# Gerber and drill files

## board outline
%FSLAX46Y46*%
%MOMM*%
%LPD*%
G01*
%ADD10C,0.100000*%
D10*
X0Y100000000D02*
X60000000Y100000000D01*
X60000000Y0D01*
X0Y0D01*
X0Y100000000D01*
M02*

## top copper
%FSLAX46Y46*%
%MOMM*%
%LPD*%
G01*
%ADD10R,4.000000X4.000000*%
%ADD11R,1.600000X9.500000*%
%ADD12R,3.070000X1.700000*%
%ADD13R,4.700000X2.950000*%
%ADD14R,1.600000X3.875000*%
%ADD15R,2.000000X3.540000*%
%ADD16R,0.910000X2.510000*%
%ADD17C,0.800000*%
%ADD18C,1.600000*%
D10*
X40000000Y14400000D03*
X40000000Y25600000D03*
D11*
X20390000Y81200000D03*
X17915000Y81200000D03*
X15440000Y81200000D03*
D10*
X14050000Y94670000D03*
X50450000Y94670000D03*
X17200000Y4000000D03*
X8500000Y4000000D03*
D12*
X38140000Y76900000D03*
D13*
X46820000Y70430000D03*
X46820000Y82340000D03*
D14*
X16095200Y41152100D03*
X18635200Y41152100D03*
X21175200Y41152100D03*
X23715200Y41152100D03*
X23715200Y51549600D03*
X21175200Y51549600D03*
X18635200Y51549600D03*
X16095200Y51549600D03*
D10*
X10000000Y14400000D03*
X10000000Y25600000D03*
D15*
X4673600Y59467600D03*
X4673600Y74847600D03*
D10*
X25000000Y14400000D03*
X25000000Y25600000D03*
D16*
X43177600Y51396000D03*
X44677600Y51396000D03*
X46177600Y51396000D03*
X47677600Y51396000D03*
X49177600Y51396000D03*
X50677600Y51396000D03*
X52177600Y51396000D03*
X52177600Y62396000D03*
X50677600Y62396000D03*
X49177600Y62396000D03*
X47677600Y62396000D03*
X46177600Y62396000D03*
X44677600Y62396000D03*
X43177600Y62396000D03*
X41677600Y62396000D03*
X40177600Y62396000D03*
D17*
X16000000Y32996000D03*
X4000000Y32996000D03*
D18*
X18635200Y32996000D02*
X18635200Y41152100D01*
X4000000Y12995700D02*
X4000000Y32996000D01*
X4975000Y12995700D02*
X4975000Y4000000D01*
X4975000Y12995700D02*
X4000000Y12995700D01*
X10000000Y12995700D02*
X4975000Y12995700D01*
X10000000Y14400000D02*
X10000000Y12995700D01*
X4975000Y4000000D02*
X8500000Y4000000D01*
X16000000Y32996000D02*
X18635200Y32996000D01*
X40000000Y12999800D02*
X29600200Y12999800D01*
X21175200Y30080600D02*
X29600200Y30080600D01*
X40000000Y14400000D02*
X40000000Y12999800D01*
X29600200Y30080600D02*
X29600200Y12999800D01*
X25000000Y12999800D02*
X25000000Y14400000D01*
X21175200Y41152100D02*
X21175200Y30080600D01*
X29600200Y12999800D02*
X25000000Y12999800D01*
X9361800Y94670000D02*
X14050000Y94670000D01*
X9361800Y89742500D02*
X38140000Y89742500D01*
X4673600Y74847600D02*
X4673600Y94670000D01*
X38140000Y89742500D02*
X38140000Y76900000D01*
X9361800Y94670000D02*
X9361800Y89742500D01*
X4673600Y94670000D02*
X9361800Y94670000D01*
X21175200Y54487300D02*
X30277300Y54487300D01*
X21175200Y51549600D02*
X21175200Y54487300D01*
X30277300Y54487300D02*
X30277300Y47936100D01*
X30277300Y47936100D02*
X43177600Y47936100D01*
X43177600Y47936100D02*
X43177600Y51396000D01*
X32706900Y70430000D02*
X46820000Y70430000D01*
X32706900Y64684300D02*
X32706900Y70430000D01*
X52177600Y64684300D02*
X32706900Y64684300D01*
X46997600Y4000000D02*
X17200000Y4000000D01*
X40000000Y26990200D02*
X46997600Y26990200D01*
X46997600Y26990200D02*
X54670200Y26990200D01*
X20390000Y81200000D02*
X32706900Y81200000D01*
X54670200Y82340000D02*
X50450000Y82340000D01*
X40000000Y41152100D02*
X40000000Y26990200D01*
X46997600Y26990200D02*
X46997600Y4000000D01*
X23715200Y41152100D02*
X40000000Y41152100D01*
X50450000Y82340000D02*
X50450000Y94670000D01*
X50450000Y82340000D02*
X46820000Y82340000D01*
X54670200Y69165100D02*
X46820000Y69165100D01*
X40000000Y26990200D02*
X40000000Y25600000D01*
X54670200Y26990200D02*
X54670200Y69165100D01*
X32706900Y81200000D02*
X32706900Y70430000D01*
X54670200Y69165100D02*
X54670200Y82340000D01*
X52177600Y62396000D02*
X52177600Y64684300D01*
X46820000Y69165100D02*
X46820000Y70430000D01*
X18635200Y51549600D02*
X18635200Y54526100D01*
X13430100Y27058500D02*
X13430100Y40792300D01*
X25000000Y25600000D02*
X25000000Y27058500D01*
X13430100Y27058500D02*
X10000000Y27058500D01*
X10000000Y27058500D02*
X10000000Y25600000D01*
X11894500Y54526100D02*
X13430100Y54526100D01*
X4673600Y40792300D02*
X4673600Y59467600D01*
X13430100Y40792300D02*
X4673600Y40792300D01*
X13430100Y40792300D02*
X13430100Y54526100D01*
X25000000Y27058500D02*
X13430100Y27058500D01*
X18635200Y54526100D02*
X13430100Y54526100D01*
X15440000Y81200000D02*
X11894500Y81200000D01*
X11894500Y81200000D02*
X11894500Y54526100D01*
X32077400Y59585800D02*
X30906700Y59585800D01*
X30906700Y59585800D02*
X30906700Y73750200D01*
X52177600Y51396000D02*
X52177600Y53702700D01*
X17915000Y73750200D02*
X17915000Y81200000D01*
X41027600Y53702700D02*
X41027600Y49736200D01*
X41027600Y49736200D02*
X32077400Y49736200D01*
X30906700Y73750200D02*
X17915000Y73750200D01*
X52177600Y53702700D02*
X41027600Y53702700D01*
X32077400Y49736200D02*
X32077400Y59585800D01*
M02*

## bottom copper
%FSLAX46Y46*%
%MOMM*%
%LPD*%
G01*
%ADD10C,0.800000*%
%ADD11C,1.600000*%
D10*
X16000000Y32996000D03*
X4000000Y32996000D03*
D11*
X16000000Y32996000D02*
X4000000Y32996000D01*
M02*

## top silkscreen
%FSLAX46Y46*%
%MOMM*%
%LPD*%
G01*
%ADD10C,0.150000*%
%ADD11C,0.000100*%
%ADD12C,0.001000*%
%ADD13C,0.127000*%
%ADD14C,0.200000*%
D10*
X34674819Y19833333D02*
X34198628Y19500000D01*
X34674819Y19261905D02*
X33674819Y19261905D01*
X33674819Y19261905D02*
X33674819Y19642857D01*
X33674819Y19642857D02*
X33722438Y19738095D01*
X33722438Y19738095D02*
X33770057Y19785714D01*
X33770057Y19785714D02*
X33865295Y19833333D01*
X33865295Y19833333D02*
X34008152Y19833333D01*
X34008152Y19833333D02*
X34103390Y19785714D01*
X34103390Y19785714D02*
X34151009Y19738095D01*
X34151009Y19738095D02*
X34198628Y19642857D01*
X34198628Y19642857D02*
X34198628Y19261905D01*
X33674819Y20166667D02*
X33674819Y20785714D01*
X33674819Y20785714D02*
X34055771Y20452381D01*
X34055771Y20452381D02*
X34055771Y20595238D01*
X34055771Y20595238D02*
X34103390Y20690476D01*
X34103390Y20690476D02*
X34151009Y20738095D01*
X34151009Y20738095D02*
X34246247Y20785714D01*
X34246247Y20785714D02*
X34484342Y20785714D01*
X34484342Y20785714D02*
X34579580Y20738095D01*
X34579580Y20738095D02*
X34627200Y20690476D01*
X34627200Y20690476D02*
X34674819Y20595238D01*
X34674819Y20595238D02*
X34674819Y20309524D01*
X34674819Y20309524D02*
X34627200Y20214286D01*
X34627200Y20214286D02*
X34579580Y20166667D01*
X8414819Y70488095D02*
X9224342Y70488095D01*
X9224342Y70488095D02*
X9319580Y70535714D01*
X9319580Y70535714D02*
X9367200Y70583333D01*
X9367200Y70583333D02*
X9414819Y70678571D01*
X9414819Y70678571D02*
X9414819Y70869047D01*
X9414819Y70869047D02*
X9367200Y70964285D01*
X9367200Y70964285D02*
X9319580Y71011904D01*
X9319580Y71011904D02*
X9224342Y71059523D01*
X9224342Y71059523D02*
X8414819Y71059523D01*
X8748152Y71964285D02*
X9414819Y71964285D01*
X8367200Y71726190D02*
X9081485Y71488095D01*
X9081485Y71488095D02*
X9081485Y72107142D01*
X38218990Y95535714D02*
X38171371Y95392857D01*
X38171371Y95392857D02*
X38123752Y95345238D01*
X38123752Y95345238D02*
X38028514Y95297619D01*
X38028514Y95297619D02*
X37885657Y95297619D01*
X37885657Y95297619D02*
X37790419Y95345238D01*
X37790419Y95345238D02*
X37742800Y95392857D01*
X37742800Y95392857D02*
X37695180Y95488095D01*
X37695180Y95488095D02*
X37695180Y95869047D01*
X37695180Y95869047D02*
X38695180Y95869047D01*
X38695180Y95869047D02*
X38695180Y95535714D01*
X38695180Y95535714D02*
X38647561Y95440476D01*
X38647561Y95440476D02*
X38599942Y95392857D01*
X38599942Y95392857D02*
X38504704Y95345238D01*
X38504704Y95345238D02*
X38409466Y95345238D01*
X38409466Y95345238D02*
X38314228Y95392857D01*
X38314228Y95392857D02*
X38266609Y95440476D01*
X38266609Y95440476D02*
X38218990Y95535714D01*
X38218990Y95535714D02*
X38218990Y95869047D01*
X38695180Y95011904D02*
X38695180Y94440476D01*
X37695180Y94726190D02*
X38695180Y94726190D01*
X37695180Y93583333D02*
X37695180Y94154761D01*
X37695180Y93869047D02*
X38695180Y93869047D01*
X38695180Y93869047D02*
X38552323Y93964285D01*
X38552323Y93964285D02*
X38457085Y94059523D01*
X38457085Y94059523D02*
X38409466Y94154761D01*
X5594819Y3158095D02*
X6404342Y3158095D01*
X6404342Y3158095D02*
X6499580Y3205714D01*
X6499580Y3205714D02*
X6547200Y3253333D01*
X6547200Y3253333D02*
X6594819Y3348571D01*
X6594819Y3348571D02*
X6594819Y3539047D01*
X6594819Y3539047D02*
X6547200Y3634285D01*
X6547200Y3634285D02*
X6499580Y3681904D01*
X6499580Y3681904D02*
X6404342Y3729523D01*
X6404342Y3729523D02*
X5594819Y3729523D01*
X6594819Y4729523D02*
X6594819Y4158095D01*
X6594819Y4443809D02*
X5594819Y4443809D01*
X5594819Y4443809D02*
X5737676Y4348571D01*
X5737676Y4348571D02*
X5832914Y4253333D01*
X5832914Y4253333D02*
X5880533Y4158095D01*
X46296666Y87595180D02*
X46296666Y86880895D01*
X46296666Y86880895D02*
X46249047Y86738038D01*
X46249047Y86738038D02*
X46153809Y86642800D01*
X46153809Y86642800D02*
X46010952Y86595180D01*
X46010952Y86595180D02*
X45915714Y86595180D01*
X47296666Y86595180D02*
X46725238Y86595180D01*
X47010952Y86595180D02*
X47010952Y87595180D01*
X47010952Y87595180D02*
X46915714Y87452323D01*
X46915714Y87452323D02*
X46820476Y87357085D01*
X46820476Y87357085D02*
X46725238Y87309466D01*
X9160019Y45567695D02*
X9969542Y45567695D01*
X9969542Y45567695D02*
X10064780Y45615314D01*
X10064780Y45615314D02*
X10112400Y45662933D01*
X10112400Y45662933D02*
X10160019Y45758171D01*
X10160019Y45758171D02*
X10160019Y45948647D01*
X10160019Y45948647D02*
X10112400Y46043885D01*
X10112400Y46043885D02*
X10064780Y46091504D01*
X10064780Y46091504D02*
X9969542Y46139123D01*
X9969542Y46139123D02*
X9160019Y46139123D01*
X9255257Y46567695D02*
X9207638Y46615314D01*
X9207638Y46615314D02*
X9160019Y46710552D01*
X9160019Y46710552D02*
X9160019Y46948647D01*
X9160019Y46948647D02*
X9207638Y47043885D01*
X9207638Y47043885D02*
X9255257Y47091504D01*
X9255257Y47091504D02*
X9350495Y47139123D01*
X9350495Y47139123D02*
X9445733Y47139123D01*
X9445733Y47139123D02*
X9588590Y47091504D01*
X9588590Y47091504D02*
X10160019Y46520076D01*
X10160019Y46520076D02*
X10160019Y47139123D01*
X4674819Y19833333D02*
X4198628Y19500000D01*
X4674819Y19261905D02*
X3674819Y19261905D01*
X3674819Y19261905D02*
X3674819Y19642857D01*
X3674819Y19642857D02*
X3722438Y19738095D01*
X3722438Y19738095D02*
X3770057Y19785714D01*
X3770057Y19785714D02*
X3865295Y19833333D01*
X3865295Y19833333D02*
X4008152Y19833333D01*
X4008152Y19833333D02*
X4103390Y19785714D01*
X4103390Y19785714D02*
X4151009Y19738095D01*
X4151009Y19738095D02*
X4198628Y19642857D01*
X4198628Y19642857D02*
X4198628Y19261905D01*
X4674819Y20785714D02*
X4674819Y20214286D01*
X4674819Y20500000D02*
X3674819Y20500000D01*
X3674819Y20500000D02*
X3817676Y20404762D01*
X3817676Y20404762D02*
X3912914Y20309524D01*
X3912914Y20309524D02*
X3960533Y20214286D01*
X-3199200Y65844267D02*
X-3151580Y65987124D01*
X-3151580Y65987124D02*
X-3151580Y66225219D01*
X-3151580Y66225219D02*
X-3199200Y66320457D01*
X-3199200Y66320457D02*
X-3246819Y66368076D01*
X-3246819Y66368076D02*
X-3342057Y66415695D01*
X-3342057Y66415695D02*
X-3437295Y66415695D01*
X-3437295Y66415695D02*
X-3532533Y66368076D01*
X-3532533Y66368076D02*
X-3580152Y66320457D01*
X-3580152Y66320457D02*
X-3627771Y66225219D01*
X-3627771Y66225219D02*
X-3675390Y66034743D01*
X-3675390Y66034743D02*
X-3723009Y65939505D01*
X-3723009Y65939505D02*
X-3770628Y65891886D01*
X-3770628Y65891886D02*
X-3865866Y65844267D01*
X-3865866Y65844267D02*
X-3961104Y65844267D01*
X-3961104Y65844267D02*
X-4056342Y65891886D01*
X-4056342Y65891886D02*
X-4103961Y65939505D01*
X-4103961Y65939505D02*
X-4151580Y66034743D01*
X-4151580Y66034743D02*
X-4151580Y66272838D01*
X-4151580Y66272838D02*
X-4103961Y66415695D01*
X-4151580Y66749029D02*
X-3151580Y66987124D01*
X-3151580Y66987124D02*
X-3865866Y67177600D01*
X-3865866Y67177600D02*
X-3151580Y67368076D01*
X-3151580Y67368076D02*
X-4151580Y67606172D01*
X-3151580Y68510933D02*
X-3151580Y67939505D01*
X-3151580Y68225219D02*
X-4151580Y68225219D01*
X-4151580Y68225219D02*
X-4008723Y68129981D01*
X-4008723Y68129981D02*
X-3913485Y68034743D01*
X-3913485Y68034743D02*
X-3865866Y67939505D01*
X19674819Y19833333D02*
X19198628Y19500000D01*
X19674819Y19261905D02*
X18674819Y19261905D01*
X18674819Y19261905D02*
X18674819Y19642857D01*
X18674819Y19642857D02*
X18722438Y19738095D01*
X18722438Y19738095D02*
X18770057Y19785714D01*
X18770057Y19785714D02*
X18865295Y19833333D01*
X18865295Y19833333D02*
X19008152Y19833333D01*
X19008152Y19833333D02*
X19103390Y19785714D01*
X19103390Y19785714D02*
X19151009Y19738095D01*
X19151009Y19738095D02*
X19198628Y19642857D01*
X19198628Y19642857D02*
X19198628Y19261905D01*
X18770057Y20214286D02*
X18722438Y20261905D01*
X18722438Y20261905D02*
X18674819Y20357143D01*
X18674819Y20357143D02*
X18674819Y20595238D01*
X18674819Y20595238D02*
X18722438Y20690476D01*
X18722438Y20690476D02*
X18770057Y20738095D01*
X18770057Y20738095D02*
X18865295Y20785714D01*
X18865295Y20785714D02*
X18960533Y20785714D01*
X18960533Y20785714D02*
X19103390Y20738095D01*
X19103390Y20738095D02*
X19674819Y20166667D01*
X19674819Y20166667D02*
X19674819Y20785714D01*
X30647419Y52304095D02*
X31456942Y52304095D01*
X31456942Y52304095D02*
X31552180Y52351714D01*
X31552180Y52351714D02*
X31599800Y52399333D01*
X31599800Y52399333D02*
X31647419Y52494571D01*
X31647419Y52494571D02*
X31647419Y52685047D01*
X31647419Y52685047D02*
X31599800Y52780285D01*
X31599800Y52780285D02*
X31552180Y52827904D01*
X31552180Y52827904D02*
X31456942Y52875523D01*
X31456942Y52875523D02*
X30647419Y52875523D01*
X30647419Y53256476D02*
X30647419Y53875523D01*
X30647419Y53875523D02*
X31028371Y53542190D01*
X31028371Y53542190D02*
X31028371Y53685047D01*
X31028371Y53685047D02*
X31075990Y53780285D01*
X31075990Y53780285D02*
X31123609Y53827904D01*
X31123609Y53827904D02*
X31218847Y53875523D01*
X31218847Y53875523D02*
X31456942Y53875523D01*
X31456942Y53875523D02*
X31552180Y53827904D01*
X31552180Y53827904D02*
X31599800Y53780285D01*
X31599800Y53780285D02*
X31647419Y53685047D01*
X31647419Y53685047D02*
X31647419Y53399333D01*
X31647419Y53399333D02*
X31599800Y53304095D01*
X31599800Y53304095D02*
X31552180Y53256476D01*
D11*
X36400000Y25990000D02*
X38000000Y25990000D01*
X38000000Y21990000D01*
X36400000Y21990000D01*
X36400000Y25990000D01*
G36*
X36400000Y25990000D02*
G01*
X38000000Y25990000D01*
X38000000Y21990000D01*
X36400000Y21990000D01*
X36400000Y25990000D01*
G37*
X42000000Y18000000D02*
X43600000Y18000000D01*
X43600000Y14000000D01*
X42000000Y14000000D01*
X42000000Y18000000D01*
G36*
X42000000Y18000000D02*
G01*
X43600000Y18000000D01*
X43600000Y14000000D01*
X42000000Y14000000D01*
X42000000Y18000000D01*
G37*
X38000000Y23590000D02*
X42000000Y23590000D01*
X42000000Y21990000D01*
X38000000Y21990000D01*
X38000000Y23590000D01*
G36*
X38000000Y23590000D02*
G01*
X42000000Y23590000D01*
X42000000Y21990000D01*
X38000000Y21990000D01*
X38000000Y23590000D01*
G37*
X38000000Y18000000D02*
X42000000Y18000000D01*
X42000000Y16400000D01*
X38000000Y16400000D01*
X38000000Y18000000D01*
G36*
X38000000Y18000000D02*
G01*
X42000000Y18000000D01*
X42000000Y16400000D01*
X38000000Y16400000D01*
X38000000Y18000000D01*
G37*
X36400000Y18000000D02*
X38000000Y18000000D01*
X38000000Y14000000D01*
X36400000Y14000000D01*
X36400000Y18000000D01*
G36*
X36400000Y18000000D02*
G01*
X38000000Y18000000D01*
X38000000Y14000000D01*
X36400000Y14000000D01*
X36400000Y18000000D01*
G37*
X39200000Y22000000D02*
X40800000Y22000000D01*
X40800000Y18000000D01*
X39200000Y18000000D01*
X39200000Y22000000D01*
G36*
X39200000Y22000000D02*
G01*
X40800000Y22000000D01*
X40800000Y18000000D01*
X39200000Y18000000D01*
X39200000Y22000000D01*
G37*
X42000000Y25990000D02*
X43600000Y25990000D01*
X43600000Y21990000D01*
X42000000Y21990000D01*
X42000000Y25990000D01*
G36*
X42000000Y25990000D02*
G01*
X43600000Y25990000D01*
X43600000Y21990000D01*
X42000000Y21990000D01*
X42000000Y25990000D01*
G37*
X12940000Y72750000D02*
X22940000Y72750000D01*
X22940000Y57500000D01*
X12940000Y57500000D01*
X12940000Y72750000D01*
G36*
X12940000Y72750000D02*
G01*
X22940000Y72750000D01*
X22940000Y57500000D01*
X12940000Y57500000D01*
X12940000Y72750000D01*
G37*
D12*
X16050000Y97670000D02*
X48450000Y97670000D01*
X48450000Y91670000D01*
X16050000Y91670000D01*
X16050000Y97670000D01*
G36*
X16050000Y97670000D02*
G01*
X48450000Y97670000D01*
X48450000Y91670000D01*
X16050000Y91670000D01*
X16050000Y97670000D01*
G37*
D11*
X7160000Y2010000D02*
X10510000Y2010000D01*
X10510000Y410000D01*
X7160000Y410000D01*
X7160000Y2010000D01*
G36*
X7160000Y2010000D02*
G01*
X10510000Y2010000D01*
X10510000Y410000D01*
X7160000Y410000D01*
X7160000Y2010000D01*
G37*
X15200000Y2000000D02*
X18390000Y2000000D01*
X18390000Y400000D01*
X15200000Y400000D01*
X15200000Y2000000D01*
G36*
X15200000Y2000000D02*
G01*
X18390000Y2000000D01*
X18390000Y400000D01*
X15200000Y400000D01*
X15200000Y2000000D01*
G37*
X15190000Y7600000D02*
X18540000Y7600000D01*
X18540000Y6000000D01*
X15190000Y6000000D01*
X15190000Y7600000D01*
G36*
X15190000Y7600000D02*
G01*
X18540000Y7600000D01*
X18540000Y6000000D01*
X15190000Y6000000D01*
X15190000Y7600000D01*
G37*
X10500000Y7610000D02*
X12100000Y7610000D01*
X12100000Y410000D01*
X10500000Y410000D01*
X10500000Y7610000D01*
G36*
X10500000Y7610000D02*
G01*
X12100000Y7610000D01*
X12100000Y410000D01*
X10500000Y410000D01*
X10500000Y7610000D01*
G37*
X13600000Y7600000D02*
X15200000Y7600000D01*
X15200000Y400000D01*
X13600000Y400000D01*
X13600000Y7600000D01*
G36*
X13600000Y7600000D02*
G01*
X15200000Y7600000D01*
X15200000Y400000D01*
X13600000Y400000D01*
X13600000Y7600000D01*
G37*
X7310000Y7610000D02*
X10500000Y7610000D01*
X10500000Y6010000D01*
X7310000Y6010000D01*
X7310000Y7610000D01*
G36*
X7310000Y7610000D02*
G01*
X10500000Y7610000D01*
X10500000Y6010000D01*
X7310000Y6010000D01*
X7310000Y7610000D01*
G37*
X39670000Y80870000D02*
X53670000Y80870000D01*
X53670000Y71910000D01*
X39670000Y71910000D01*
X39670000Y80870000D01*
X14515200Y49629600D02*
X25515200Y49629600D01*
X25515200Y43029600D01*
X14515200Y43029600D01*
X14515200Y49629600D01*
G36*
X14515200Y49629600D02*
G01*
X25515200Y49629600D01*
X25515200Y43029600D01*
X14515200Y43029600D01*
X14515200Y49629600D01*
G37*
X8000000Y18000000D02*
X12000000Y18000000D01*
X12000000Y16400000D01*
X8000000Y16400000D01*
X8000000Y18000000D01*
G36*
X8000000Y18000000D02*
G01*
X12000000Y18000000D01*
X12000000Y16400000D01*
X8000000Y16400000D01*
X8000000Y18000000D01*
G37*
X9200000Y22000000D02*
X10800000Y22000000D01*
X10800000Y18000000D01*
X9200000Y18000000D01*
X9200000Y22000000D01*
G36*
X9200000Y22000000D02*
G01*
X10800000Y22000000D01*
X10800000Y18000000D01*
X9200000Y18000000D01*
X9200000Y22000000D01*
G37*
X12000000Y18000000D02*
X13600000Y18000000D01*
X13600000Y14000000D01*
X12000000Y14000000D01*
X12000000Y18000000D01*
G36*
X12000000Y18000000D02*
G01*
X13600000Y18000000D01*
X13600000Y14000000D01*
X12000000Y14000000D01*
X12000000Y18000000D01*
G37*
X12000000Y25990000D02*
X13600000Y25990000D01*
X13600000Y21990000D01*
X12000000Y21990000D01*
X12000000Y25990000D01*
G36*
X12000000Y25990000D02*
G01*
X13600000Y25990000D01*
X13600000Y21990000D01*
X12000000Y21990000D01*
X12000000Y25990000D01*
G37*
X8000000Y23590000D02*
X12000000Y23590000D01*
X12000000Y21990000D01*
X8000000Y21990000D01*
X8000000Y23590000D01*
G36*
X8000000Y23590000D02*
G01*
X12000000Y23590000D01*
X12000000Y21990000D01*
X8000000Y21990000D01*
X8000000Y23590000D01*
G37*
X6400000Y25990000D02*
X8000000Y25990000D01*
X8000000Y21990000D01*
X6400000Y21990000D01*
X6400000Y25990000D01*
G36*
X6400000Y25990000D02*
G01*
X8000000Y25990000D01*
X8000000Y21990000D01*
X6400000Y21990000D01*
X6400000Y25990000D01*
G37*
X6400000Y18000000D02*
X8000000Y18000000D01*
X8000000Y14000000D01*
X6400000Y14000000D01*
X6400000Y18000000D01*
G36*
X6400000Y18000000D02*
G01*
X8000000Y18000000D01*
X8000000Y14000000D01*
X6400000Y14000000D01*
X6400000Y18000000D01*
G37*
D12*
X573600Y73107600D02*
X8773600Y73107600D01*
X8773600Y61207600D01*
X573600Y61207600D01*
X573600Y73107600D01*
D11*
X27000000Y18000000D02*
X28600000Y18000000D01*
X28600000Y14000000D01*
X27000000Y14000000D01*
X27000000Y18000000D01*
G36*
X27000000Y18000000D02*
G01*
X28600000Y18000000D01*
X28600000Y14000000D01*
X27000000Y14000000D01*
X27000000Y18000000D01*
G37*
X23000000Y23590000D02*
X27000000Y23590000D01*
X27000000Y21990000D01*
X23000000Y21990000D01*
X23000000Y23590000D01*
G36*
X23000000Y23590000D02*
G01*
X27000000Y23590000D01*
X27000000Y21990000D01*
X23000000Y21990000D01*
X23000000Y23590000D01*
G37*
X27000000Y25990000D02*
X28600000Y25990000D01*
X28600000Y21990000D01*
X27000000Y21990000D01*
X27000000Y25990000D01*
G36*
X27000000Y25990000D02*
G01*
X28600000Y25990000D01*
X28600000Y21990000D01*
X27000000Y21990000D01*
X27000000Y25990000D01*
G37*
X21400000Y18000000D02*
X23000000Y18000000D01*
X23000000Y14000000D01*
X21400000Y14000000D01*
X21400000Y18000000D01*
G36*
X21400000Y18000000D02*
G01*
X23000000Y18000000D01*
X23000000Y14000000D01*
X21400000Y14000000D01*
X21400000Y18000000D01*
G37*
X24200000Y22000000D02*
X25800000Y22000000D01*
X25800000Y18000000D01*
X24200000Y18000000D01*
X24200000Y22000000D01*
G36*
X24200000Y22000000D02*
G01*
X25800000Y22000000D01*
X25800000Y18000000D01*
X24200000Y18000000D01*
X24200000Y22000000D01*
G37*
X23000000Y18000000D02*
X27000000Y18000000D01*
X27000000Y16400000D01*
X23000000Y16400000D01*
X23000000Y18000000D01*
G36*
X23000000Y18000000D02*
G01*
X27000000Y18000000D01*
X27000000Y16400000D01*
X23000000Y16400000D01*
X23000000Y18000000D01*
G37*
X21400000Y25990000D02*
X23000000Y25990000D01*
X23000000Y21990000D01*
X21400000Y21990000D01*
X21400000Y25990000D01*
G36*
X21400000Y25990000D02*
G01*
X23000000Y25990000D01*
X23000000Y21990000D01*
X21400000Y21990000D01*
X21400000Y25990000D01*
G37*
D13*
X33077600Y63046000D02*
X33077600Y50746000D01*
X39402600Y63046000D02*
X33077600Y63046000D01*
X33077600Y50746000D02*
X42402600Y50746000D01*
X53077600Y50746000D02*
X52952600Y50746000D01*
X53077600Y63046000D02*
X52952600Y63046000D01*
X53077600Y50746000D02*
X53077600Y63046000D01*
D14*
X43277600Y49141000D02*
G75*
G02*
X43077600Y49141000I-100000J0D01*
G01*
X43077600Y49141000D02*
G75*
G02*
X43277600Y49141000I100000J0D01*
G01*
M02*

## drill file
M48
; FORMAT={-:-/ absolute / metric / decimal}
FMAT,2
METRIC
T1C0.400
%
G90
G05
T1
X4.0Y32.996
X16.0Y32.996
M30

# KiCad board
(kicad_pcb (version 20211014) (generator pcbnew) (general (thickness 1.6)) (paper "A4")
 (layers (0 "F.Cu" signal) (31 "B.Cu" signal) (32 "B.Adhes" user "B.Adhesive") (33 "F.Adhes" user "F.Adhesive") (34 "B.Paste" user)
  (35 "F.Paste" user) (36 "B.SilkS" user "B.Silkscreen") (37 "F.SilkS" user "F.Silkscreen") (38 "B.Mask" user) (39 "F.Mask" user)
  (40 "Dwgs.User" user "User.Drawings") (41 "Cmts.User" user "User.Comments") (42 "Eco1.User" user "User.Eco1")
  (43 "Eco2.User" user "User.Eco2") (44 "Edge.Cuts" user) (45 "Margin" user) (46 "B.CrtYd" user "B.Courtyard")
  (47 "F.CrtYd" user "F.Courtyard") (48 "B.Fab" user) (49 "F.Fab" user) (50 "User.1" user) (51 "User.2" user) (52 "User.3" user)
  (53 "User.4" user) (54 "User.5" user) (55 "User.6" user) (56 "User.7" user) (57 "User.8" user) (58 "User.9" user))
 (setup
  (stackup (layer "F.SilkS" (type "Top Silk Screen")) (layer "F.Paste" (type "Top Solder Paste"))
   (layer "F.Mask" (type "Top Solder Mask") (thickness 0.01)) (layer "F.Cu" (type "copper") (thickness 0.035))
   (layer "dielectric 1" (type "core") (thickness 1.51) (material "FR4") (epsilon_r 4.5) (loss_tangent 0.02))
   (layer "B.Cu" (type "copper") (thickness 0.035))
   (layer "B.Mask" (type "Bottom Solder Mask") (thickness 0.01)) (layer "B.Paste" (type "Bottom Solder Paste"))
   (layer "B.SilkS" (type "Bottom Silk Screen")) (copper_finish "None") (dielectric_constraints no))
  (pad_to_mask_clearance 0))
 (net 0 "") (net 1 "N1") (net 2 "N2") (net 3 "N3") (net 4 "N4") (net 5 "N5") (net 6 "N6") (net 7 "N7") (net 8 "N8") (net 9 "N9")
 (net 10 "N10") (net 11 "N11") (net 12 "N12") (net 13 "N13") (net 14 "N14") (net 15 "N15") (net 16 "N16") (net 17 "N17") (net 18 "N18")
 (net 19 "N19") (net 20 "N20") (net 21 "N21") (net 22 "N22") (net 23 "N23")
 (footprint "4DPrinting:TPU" (layer "F.Cu") (at 40 -20 90)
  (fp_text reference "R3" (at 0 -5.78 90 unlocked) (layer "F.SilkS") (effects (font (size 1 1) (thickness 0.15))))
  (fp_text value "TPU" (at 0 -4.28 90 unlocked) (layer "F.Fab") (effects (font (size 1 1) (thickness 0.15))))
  (fp_rect (start 1.99 -3.6) (end 5.99 -2) (layer "F.SilkS") (width 0.0001) (fill solid))
  (fp_rect (start -6 2) (end -2 3.6) (layer "F.SilkS") (width 0.0001) (fill solid))
  (fp_rect (start 1.99 -2) (end 3.59 2) (layer "F.SilkS") (width 0.0001) (fill solid))
  (fp_rect (start -3.6 -2) (end -2 2) (layer "F.SilkS") (width 0.0001) (fill solid))
  (fp_rect (start -6 -3.6) (end -2 -2) (layer "F.SilkS") (width 0.0001) (fill solid))
  (fp_rect (start -2 -0.8) (end 2 0.8) (layer "F.SilkS") (width 0.0001) (fill solid))
  (fp_rect (start 1.99 2) (end 5.99 3.6) (layer "F.SilkS") (width 0.0001) (fill solid))
  (pad "1" smd rect (at -5.6 0 90) (size 4 4) (layers "F.Cu" "F.Paste" "F.Mask") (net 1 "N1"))
  (pad "2" smd rect (at 5.6 0 90) (size 4 4) (layers "F.Cu" "F.Paste" "F.Mask") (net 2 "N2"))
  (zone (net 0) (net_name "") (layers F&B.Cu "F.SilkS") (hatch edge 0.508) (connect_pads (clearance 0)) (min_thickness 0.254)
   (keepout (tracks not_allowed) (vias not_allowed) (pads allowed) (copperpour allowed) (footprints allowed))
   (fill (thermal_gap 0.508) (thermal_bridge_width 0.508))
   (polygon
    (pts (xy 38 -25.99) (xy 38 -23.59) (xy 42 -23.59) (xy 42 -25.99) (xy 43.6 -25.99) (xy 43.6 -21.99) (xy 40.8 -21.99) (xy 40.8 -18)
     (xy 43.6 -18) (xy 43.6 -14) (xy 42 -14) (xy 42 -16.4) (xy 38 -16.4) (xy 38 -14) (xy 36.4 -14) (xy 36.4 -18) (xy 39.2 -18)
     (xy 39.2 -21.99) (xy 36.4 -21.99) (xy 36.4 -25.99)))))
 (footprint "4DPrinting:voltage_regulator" (layer "F.Cu") (at 17.99 -71.23 90)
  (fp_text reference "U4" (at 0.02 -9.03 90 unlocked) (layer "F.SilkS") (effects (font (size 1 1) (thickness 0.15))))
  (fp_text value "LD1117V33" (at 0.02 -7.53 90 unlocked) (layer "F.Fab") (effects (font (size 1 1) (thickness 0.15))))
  (fp_rect (start -13.73 -5.05) (end 1.52 4.95) (layer "F.SilkS") (width 0.0001) (fill solid))
  (pad "1" smd rect (at 9.97 2.4 90) (size 9.5 1.6) (layers "F.Cu" "F.Paste" "F.Mask") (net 2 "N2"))
  (pad "2" smd rect (at 9.97 -0.075 90) (size 9.5 1.6) (layers "F.Cu" "F.Paste" "F.Mask") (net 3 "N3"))
  (pad "3" smd rect (at 9.97 -2.55 90) (size 9.5 1.6) (layers "F.Cu" "F.Paste" "F.Mask") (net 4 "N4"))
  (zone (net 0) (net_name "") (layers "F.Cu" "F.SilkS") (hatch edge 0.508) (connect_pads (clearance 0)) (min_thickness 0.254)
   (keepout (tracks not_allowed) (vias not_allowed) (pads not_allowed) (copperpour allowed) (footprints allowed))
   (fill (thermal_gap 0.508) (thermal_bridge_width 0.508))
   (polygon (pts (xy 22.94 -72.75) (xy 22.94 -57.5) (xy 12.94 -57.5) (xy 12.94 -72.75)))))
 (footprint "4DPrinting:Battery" (layer "F.Cu") (at 32.25 -94.67 -90)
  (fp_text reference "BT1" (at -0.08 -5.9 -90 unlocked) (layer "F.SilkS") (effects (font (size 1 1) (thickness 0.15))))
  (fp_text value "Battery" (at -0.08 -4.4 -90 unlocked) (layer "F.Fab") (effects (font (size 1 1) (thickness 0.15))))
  (fp_rect (start -3 -16.2) (end 3 16.2) (layer "F.SilkS") (width 0.001) (fill solid))
  (pad "1" smd rect (at 0 18.2 270) (size 4 4) (layers "F.Cu" "F.Paste" "F.Mask") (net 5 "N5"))
  (pad "2" smd rect (at 0 -18.2 270) (size 4 4) (layers "F.Cu" "F.Paste" "F.Mask") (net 2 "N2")))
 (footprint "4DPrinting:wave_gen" (layer "F.Cu") (at 12.85 -4 90)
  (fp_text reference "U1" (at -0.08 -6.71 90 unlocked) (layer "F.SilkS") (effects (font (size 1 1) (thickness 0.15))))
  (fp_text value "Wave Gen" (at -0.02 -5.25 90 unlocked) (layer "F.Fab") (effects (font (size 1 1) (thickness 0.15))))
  (fp_rect (start -3.59 -2.34) (end -1.99 -5.69) (layer "F.SilkS") (width 0.0001) (fill solid))
  (fp_rect (start -2 2.35) (end -3.6 5.54) (layer "F.SilkS") (width 0.0001) (fill solid))
  (fp_rect (start 3.6 2.34) (end 2 5.69) (layer "F.SilkS") (width 0.0001) (fill solid))
  (fp_rect (start 3.61 -0.75) (end -3.59 -2.35) (layer "F.SilkS") (width 0.0001) (fill solid))
  (fp_rect (start -3.6 0.75) (end 3.6 2.35) (layer "F.SilkS") (width 0.0001) (fill solid))
  (fp_rect (start 2.01 -2.35) (end 3.61 -5.54) (layer "F.SilkS") (width 0.0001) (fill solid))
  (pad "1" smd rect (at 0 4.35 90) (size 4 4) (layers "F.Cu" "F.Paste" "F.Mask") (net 2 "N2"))
  (pad "2" smd rect (at 0 -4.35 270) (size 4 4) (layers "F.Cu" "F.Paste" "F.Mask") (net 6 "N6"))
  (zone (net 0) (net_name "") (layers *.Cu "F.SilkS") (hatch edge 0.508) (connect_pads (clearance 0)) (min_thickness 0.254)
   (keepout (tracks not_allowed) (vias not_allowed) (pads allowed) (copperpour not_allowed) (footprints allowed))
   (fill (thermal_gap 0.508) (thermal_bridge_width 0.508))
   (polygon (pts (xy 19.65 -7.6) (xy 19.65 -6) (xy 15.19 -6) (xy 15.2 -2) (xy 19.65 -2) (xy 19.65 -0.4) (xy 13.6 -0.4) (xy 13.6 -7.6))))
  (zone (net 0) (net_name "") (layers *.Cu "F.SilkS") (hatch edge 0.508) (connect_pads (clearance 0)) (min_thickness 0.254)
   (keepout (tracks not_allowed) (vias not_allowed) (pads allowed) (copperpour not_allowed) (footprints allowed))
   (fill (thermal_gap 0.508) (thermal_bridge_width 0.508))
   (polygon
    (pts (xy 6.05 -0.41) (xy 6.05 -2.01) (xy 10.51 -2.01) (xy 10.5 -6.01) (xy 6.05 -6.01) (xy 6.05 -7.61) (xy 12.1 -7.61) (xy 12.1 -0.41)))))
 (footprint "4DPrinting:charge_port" (layer "F.Cu") (at 46.67 -76.39)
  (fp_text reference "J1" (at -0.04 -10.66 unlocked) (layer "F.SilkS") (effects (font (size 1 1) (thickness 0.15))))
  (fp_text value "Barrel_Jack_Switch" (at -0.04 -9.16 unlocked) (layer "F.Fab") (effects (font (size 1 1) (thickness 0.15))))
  (fp_rect (start -7 -4.48) (end 7 4.48) (layer "F.SilkS") (width 0.0001) (fill none))
  (pad "1" smd rect (at -8.53 -0.51 180) (size 3.07 1.7) (layers "F.Cu" "F.Paste" "F.Mask") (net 5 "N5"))
  (pad "2" smd rect (at 0.15 5.96 180) (size 4.7 2.95) (layers "F.Cu" "F.Paste" "F.Mask") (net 2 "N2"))
  (pad "3" smd rect (at 0.15 -5.95 180) (size 4.7 2.95) (layers "F.Cu" "F.Paste" "F.Mask") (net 2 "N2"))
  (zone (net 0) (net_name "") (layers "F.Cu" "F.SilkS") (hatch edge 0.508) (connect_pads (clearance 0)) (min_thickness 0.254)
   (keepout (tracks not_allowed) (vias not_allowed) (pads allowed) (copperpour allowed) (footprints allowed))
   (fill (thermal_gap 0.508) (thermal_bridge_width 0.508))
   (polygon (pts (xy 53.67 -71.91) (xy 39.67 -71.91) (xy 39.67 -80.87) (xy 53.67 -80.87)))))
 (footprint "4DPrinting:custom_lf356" (layer "F.Cu") (at 20.0152 -46.3296 90)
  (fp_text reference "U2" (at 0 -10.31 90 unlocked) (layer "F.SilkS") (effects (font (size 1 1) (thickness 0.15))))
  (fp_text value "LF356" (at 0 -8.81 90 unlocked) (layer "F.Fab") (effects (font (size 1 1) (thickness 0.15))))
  (fp_rect (start -3.3 -5.5) (end 3.3 5.5) (layer "F.SilkS") (width 0.0001) (fill solid))
  (pad "1" smd rect (at -5.1775 -3.92 90) (size 3.875 1.6) (layers "F.Cu" "F.Paste" "F.Mask") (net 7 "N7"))
  (pad "2" smd rect (at -5.1775 -1.38 90) (size 3.875 1.6) (layers "F.Cu" "F.Paste" "F.Mask") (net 6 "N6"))
  (pad "3" smd rect (at -5.1775 1.16 90) (size 3.875 1.6) (layers "F.Cu" "F.Paste" "F.Mask") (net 1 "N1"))
  (pad "4" smd rect (at -5.1775 3.7 90) (size 3.875 1.6) (layers "F.Cu" "F.Paste" "F.Mask") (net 2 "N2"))
  (pad "5" smd rect (at 5.22 3.7 90) (size 3.875 1.6) (layers "F.Cu" "F.Paste" "F.Mask") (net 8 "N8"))
  (pad "6" smd rect (at 5.22 1.16 90) (size 3.875 1.6) (layers "F.Cu" "F.Paste" "F.Mask") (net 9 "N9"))
  (pad "7" smd rect (at 5.22 -1.38 90) (size 3.875 1.6) (layers "F.Cu" "F.Paste" "F.Mask") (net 4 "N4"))
  (pad "8" smd rect (at 5.22 -3.92 90) (size 3.875 1.6) (layers "F.Cu" "F.Paste" "F.Mask") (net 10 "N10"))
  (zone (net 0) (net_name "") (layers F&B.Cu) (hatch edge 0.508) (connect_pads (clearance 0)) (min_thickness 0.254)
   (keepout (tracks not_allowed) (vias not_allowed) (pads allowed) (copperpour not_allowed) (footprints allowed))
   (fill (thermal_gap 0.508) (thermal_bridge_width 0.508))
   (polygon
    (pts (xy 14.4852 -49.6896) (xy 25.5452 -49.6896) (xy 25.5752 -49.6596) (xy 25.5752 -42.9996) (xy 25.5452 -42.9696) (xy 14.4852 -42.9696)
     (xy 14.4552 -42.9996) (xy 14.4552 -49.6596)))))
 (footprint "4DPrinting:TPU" (layer "F.Cu") (at 10 -20 90)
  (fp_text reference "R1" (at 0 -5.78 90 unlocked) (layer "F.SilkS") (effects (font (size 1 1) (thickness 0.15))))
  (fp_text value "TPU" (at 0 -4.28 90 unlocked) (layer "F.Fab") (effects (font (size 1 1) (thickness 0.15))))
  (fp_rect (start -3.6 -2) (end -2 2) (layer "F.SilkS") (width 0.0001) (fill solid))
  (fp_rect (start -2 -0.8) (end 2 0.8) (layer "F.SilkS") (width 0.0001) (fill solid))
  (fp_rect (start -6 2) (end -2 3.6) (layer "F.SilkS") (width 0.0001) (fill solid))
  (fp_rect (start 1.99 2) (end 5.99 3.6) (layer "F.SilkS") (width 0.0001) (fill solid))
  (fp_rect (start 1.99 -2) (end 3.59 2) (layer "F.SilkS") (width 0.0001) (fill solid))
  (fp_rect (start 1.99 -3.6) (end 5.99 -2) (layer "F.SilkS") (width 0.0001) (fill solid))
  (fp_rect (start -6 -3.6) (end -2 -2) (layer "F.SilkS") (width 0.0001) (fill solid))
  (pad "1" smd rect (at -5.6 0 90) (size 4 4) (layers "F.Cu" "F.Paste" "F.Mask") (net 6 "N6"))
  (pad "2" smd rect (at 5.6 0 90) (size 4 4) (layers "F.Cu" "F.Paste" "F.Mask") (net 4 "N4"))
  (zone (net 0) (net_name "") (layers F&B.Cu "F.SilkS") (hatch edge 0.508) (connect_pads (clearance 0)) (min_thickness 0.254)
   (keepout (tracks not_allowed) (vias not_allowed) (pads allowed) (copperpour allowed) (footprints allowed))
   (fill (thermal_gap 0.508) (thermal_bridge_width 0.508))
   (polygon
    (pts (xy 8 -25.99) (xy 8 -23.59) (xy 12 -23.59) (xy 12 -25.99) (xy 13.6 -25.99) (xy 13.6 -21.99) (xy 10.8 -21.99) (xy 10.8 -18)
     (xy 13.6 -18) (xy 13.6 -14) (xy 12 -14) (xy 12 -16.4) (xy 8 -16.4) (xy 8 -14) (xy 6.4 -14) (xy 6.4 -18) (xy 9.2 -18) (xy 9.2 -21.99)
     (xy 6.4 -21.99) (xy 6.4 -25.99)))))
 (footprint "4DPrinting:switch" (layer "F.Cu") (at 4.6736 -67.1576 90)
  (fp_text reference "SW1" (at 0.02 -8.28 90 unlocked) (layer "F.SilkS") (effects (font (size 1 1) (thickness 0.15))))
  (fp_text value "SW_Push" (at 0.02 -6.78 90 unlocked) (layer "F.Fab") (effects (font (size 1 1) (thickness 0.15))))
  (fp_rect (start -5.95 4.1) (end 5.95 -4.1) (layer "F.SilkS") (width 0.001) (fill none))
  (pad "1" smd rect (at -7.69 0 90) (size 3.54 2) (layers "F.Cu" "F.Paste" "F.Mask") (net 4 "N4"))
  (pad "2" smd rect (at 7.69 0 90) (size 3.54 2) (layers "F.Cu" "F.Paste" "F.Mask") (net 5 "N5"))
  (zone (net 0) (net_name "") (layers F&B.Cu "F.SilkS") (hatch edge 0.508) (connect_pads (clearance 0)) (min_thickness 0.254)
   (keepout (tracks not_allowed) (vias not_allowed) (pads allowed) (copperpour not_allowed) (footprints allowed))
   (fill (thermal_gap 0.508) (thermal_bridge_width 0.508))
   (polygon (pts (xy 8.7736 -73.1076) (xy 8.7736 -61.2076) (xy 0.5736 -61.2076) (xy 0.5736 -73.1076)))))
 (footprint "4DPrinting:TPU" (layer "F.Cu") (at 25 -20 90)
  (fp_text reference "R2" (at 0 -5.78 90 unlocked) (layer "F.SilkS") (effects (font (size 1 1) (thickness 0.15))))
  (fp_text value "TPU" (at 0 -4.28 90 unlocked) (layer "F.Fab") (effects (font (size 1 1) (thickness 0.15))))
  (fp_rect (start -6 2) (end -2 3.6) (layer "F.SilkS") (width 0.0001) (fill solid))
  (fp_rect (start 1.99 -2) (end 3.59 2) (layer "F.SilkS") (width 0.0001) (fill solid))
  (fp_rect (start 1.99 2) (end 5.99 3.6) (layer "F.SilkS") (width 0.0001) (fill solid))
  (fp_rect (start -6 -3.6) (end -2 -2) (layer "F.SilkS") (width 0.0001) (fill solid))
  (fp_rect (start -2 -0.8) (end 2 0.8) (layer "F.SilkS") (width 0.0001) (fill solid))
  (fp_rect (start -3.6 -2) (end -2 2) (layer "F.SilkS") (width 0.0001) (fill solid))
  (fp_rect (start 1.99 -3.6) (end 5.99 -2) (layer "F.SilkS") (width 0.0001) (fill solid))
  (pad "1" smd rect (at -5.6 0 90) (size 4 4) (layers "F.Cu" "F.Paste" "F.Mask") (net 1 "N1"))
  (pad "2" smd rect (at 5.6 0 90) (size 4 4) (layers "F.Cu" "F.Paste" "F.Mask") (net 4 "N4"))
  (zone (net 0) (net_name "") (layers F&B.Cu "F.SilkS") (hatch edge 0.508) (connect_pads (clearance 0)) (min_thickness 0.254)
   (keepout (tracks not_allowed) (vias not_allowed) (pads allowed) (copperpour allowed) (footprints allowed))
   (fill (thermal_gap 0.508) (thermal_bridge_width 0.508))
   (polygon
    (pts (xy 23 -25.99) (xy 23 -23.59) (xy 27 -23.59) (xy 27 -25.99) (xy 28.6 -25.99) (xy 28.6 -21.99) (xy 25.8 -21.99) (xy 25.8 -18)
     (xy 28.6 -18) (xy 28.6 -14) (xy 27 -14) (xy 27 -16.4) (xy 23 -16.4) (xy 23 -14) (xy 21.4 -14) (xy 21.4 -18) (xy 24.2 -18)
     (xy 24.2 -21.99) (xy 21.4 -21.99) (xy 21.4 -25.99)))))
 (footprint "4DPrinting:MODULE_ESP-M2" (layer "F.Cu") (at 43.0776 -56.896 90)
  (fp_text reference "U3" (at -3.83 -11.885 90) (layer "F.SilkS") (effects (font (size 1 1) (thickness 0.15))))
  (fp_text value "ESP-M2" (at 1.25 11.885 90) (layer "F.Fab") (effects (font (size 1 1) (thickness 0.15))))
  (fp_line (start 6.15 -10) (end -6.15 -10) (layer "F.SilkS") (width 0.127))
  (fp_line (start 6.15 -3.675) (end 6.15 -10) (layer "F.SilkS") (width 0.127))
  (fp_line (start -6.15 -10) (end -6.15 -0.675) (layer "F.SilkS") (width 0.127))
  (fp_line (start -6.15 10) (end -6.15 9.875) (layer "F.SilkS") (width 0.127))
  (fp_line (start 6.15 10) (end 6.15 9.875) (layer "F.SilkS") (width 0.127))
  (fp_line (start -6.15 10) (end 6.15 10) (layer "F.SilkS") (width 0.127))
  (fp_circle (center -7.755 0.1) (end -7.655 0.1) (layer "F.SilkS") (width 0.2) (fill none))
  (pad "1" smd rect (at -5.5 0.1 90) (size 2.51 0.91) (layers "F.Cu" "F.Paste" "F.Mask") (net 9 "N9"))
  (pad "2" smd rect (at -5.5 1.6 90) (size 2.51 0.91) (layers "F.Cu" "F.Paste" "F.Mask") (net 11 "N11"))
  (pad "3" smd rect (at -5.5 3.1 90) (size 2.51 0.91) (layers "F.Cu" "F.Paste" "F.Mask") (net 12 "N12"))
  (pad "4" smd rect (at -5.5 4.6 90) (size 2.51 0.91) (layers "F.Cu" "F.Paste" "F.Mask") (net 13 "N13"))
  (pad "5" smd rect (at -5.5 6.1 90) (size 2.51 0.91) (layers "F.Cu" "F.Paste" "F.Mask") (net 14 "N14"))
  (pad "6" smd rect (at -5.5 7.6 90) (size 2.51 0.91) (layers "F.Cu" "F.Paste" "F.Mask") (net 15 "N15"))
  (pad "7" smd rect (at -5.5 9.1 90) (size 2.51 0.91) (layers "F.Cu" "F.Paste" "F.Mask") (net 3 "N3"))
  (pad "8" smd rect (at 5.5 9.1 90) (size 2.51 0.91) (layers "F.Cu" "F.Paste" "F.Mask") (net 2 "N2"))
  (pad "9" smd rect (at 5.5 7.6 90) (size 2.51 0.91) (layers "F.Cu" "F.Paste" "F.Mask") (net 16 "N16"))
  (pad "10" smd rect (at 5.5 6.1 90) (size 2.51 0.91) (layers "F.Cu" "F.Paste" "F.Mask") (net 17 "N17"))
  (pad "11" smd rect (at 5.5 4.6 90) (size 2.51 0.91) (layers "F.Cu" "F.Paste" "F.Mask") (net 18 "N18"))
  (pad "12" smd rect (at 5.5 3.1 90) (size 2.51 0.91) (layers "F.Cu" "F.Paste" "F.Mask") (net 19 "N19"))
  (pad "13" smd rect (at 5.5 1.6 90) (size 2.51 0.91) (layers "F.Cu" "F.Paste" "F.Mask") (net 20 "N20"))
  (pad "14" smd rect (at 5.5 0.1 90) (size 2.51 0.91) (layers "F.Cu" "F.Paste" "F.Mask") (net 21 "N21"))
  (pad "15" smd rect (at 5.5 -1.4 90) (size 2.51 0.91) (layers "F.Cu" "F.Paste" "F.Mask") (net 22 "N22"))
  (pad "16" smd rect (at 5.5 -2.9 90) (size 2.51 0.91) (layers "F.Cu" "F.Paste" "F.Mask") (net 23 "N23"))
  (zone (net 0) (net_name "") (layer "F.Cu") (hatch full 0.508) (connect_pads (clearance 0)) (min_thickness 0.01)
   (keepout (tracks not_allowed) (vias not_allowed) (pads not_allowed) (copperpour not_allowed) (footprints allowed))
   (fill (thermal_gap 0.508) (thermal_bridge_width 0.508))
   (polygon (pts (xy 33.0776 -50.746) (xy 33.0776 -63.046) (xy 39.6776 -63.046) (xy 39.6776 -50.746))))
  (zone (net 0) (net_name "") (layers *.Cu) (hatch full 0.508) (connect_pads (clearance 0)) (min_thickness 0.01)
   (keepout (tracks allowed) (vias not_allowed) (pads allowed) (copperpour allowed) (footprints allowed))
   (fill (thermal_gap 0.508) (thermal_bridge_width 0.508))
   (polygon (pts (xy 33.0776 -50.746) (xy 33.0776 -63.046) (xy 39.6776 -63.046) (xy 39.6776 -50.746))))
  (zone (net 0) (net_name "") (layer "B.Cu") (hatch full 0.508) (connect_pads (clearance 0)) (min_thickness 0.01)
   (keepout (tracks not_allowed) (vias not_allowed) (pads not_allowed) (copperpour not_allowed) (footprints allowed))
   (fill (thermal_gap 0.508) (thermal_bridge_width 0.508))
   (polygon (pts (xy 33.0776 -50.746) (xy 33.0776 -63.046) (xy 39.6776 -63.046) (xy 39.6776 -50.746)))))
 (gr_rect (start 60 -100) (end 0 0) (layer "Edge.Cuts") (width 0.1) (fill none))
 (segment (start 18.6352 -32.996) (end 18.6352 -41.1521) (width 1.6) (layer "F.Cu") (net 6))
 (segment (start 4 -12.9957) (end 4 -32.996) (width 1.6) (layer "F.Cu") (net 6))
 (segment (start 4.975 -12.9957) (end 4.975 -4) (width 1.6) (layer "F.Cu") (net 6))
 (segment (start 4.975 -12.9957) (end 4 -12.9957) (width 1.6) (layer "F.Cu") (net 6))
 (segment (start 10 -12.9957) (end 4.975 -12.9957) (width 1.6) (layer "F.Cu") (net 6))
 (segment (start 10 -14.4) (end 10 -12.9957) (width 1.6) (layer "F.Cu") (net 6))
 (segment (start 4.975 -4) (end 8.5 -4) (width 1.6) (layer "F.Cu") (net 6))
 (segment (start 16 -32.996) (end 18.6352 -32.996) (width 1.6) (layer "F.Cu") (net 6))
 (via (at 16 -32.996) (size 0.8) (drill 0.4) (layers "F.Cu" "B.Cu") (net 6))
 (via (at 4 -32.996) (size 0.8) (drill 0.4) (layers "F.Cu" "B.Cu") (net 6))
 (segment (start 16 -32.996) (end 4 -32.996) (width 1.6) (layer "B.Cu") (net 6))
 (segment (start 40 -12.9998) (end 29.6002 -12.9998) (width 1.6) (layer "F.Cu") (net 1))
 (segment (start 21.1752 -30.0806) (end 29.6002 -30.0806) (width 1.6) (layer "F.Cu") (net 1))
 (segment (start 40 -14.4) (end 40 -12.9998) (width 1.6) (layer "F.Cu") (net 1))
 (segment (start 29.6002 -30.0806) (end 29.6002 -12.9998) (width 1.6) (layer "F.Cu") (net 1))
 (segment (start 25 -12.9998) (end 25 -14.4) (width 1.6) (layer "F.Cu") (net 1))
 (segment (start 21.1752 -41.1521) (end 21.1752 -30.0806) (width 1.6) (layer "F.Cu") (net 1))
 (segment (start 29.6002 -12.9998) (end 25 -12.9998) (width 1.6) (layer "F.Cu") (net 1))
 (segment (start 9.3618 -94.67) (end 14.05 -94.67) (width 1.6) (layer "F.Cu") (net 5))
 (segment (start 9.3618 -89.7425) (end 38.14 -89.7425) (width 1.6) (layer "F.Cu") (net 5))
 (segment (start 4.6736 -74.8476) (end 4.6736 -94.67) (width 1.6) (layer "F.Cu") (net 5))
 (segment (start 38.14 -89.7425) (end 38.14 -76.9) (width 1.6) (layer "F.Cu") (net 5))
 (segment (start 9.3618 -94.67) (end 9.3618 -89.7425) (width 1.6) (layer "F.Cu") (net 5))
 (segment (start 4.6736 -94.67) (end 9.3618 -94.67) (width 1.6) (layer "F.Cu") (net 5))
 (segment (start 21.1752 -54.4873) (end 30.2773 -54.4873) (width 1.6) (layer "F.Cu") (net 9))
 (segment (start 21.1752 -51.5496) (end 21.1752 -54.4873) (width 1.6) (layer "F.Cu") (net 9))
 (segment (start 30.2773 -54.4873) (end 30.2773 -47.9361) (width 1.6) (layer "F.Cu") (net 9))
 (segment (start 30.2773 -47.9361) (end 43.1776 -47.9361) (width 1.6) (layer "F.Cu") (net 9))
 (segment (start 43.1776 -47.9361) (end 43.1776 -51.396) (width 1.6) (layer "F.Cu") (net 9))
 (segment (start 32.7069 -70.43) (end 46.82 -70.43) (width 1.6) (layer "F.Cu") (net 2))
 (segment (start 32.7069 -64.6843) (end 32.7069 -70.43) (width 1.6) (layer "F.Cu") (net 2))
 (segment (start 52.1776 -64.6843) (end 32.7069 -64.6843) (width 1.6) (layer "F.Cu") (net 2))
 (segment (start 46.9976 -4) (end 17.2 -4) (width 1.6) (layer "F.Cu") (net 2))
 (segment (start 40 -26.9902) (end 46.9976 -26.9902) (width 1.6) (layer "F.Cu") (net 2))
 (segment (start 46.9976 -26.9902) (end 54.6702 -26.9902) (width 1.6) (layer "F.Cu") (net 2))
 (segment (start 20.39 -81.2) (end 32.7069 -81.2) (width 1.6) (layer "F.Cu") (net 2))
 (segment (start 54.6702 -82.34) (end 50.45 -82.34) (width 1.6) (layer "F.Cu") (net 2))
 (segment (start 40 -41.1521) (end 40 -26.9902) (width 1.6) (layer "F.Cu") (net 2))
 (segment (start 46.9976 -26.9902) (end 46.9976 -4) (width 1.6) (layer "F.Cu") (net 2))
 (segment (start 23.7152 -41.1521) (end 40 -41.1521) (width 1.6) (layer "F.Cu") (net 2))
 (segment (start 50.45 -82.34) (end 50.45 -94.67) (width 1.6) (layer "F.Cu") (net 2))
 (segment (start 50.45 -82.34) (end 46.82 -82.34) (width 1.6) (layer "F.Cu") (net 2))
 (segment (start 54.6702 -69.1651) (end 46.82 -69.1651) (width 1.6) (layer "F.Cu") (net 2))
 (segment (start 40 -26.9902) (end 40 -25.6) (width 1.6) (layer "F.Cu") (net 2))
 (segment (start 54.6702 -26.9902) (end 54.6702 -69.1651) (width 1.6) (layer "F.Cu") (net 2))
 (segment (start 32.7069 -81.2) (end 32.7069 -70.43) (width 1.6) (layer "F.Cu") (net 2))
 (segment (start 54.6702 -69.1651) (end 54.6702 -82.34) (width 1.6) (layer "F.Cu") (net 2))
 (segment (start 52.1776 -62.396) (end 52.1776 -64.6843) (width 1.6) (layer "F.Cu") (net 2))
 (segment (start 46.82 -69.1651) (end 46.82 -70.43) (width 1.6) (layer "F.Cu") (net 2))
 (segment (start 18.6352 -51.5496) (end 18.6352 -54.5261) (width 1.6) (layer "F.Cu") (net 4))
 (segment (start 13.4301 -27.0585) (end 13.4301 -40.7923) (width 1.6) (layer "F.Cu") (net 4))
 (segment (start 25 -25.6) (end 25 -27.0585) (width 1.6) (layer "F.Cu") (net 4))
 (segment (start 13.4301 -27.0585) (end 10 -27.0585) (width 1.6) (layer "F.Cu") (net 4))
 (segment (start 10 -27.0585) (end 10 -25.6) (width 1.6) (layer "F.Cu") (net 4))
 (segment (start 11.8945 -54.5261) (end 13.4301 -54.5261) (width 1.6) (layer "F.Cu") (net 4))
 (segment (start 4.6736 -40.7923) (end 4.6736 -59.4676) (width 1.6) (layer "F.Cu") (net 4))
 (segment (start 13.4301 -40.7923) (end 4.6736 -40.7923) (width 1.6) (layer "F.Cu") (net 4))
 (segment (start 13.4301 -40.7923) (end 13.4301 -54.5261) (width 1.6) (layer "F.Cu") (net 4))
 (segment (start 25 -27.0585) (end 13.4301 -27.0585) (width 1.6) (layer "F.Cu") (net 4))
 (segment (start 18.6352 -54.5261) (end 13.4301 -54.5261) (width 1.6) (layer "F.Cu") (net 4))
 (segment (start 15.44 -81.2) (end 11.8945 -81.2) (width 1.6) (layer "F.Cu") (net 4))
 (segment (start 11.8945 -81.2) (end 11.8945 -54.5261) (width 1.6) (layer "F.Cu") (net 4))
 (segment (start 32.0774 -59.5858) (end 30.9067 -59.5858) (width 1.6) (layer "F.Cu") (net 3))
 (segment (start 30.9067 -59.5858) (end 30.9067 -73.7502) (width 1.6) (layer "F.Cu") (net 3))
 (segment (start 52.1776 -51.396) (end 52.1776 -53.7027) (width 1.6) (layer "F.Cu") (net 3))
 (segment (start 17.915 -73.7502) (end 17.915 -81.2) (width 1.6) (layer "F.Cu") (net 3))
 (segment (start 41.0276 -53.7027) (end 41.0276 -49.7362) (width 1.6) (layer "F.Cu") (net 3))
 (segment (start 41.0276 -49.7362) (end 32.0774 -49.7362) (width 1.6) (layer "F.Cu") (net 3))
 (segment (start 30.9067 -73.7502) (end 17.915 -73.7502) (width 1.6) (layer "F.Cu") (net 3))
 (segment (start 52.1776 -53.7027) (end 41.0276 -53.7027) (width 1.6) (layer "F.Cu") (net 3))
 (segment (start 32.0774 -49.7362) (end 32.0774 -59.5858) (width 1.6) (layer "F.Cu") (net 3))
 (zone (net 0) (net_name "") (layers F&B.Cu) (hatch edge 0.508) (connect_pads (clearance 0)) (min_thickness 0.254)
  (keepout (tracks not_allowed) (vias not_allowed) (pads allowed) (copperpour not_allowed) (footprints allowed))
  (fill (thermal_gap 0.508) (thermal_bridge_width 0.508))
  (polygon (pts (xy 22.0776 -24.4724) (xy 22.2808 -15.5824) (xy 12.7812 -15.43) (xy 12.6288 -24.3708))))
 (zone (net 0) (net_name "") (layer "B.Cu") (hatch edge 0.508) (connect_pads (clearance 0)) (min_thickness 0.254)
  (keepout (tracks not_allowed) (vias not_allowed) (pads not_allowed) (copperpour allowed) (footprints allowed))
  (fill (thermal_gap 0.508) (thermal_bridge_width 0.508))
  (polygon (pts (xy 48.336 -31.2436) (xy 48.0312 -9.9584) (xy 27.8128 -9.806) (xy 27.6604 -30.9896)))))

